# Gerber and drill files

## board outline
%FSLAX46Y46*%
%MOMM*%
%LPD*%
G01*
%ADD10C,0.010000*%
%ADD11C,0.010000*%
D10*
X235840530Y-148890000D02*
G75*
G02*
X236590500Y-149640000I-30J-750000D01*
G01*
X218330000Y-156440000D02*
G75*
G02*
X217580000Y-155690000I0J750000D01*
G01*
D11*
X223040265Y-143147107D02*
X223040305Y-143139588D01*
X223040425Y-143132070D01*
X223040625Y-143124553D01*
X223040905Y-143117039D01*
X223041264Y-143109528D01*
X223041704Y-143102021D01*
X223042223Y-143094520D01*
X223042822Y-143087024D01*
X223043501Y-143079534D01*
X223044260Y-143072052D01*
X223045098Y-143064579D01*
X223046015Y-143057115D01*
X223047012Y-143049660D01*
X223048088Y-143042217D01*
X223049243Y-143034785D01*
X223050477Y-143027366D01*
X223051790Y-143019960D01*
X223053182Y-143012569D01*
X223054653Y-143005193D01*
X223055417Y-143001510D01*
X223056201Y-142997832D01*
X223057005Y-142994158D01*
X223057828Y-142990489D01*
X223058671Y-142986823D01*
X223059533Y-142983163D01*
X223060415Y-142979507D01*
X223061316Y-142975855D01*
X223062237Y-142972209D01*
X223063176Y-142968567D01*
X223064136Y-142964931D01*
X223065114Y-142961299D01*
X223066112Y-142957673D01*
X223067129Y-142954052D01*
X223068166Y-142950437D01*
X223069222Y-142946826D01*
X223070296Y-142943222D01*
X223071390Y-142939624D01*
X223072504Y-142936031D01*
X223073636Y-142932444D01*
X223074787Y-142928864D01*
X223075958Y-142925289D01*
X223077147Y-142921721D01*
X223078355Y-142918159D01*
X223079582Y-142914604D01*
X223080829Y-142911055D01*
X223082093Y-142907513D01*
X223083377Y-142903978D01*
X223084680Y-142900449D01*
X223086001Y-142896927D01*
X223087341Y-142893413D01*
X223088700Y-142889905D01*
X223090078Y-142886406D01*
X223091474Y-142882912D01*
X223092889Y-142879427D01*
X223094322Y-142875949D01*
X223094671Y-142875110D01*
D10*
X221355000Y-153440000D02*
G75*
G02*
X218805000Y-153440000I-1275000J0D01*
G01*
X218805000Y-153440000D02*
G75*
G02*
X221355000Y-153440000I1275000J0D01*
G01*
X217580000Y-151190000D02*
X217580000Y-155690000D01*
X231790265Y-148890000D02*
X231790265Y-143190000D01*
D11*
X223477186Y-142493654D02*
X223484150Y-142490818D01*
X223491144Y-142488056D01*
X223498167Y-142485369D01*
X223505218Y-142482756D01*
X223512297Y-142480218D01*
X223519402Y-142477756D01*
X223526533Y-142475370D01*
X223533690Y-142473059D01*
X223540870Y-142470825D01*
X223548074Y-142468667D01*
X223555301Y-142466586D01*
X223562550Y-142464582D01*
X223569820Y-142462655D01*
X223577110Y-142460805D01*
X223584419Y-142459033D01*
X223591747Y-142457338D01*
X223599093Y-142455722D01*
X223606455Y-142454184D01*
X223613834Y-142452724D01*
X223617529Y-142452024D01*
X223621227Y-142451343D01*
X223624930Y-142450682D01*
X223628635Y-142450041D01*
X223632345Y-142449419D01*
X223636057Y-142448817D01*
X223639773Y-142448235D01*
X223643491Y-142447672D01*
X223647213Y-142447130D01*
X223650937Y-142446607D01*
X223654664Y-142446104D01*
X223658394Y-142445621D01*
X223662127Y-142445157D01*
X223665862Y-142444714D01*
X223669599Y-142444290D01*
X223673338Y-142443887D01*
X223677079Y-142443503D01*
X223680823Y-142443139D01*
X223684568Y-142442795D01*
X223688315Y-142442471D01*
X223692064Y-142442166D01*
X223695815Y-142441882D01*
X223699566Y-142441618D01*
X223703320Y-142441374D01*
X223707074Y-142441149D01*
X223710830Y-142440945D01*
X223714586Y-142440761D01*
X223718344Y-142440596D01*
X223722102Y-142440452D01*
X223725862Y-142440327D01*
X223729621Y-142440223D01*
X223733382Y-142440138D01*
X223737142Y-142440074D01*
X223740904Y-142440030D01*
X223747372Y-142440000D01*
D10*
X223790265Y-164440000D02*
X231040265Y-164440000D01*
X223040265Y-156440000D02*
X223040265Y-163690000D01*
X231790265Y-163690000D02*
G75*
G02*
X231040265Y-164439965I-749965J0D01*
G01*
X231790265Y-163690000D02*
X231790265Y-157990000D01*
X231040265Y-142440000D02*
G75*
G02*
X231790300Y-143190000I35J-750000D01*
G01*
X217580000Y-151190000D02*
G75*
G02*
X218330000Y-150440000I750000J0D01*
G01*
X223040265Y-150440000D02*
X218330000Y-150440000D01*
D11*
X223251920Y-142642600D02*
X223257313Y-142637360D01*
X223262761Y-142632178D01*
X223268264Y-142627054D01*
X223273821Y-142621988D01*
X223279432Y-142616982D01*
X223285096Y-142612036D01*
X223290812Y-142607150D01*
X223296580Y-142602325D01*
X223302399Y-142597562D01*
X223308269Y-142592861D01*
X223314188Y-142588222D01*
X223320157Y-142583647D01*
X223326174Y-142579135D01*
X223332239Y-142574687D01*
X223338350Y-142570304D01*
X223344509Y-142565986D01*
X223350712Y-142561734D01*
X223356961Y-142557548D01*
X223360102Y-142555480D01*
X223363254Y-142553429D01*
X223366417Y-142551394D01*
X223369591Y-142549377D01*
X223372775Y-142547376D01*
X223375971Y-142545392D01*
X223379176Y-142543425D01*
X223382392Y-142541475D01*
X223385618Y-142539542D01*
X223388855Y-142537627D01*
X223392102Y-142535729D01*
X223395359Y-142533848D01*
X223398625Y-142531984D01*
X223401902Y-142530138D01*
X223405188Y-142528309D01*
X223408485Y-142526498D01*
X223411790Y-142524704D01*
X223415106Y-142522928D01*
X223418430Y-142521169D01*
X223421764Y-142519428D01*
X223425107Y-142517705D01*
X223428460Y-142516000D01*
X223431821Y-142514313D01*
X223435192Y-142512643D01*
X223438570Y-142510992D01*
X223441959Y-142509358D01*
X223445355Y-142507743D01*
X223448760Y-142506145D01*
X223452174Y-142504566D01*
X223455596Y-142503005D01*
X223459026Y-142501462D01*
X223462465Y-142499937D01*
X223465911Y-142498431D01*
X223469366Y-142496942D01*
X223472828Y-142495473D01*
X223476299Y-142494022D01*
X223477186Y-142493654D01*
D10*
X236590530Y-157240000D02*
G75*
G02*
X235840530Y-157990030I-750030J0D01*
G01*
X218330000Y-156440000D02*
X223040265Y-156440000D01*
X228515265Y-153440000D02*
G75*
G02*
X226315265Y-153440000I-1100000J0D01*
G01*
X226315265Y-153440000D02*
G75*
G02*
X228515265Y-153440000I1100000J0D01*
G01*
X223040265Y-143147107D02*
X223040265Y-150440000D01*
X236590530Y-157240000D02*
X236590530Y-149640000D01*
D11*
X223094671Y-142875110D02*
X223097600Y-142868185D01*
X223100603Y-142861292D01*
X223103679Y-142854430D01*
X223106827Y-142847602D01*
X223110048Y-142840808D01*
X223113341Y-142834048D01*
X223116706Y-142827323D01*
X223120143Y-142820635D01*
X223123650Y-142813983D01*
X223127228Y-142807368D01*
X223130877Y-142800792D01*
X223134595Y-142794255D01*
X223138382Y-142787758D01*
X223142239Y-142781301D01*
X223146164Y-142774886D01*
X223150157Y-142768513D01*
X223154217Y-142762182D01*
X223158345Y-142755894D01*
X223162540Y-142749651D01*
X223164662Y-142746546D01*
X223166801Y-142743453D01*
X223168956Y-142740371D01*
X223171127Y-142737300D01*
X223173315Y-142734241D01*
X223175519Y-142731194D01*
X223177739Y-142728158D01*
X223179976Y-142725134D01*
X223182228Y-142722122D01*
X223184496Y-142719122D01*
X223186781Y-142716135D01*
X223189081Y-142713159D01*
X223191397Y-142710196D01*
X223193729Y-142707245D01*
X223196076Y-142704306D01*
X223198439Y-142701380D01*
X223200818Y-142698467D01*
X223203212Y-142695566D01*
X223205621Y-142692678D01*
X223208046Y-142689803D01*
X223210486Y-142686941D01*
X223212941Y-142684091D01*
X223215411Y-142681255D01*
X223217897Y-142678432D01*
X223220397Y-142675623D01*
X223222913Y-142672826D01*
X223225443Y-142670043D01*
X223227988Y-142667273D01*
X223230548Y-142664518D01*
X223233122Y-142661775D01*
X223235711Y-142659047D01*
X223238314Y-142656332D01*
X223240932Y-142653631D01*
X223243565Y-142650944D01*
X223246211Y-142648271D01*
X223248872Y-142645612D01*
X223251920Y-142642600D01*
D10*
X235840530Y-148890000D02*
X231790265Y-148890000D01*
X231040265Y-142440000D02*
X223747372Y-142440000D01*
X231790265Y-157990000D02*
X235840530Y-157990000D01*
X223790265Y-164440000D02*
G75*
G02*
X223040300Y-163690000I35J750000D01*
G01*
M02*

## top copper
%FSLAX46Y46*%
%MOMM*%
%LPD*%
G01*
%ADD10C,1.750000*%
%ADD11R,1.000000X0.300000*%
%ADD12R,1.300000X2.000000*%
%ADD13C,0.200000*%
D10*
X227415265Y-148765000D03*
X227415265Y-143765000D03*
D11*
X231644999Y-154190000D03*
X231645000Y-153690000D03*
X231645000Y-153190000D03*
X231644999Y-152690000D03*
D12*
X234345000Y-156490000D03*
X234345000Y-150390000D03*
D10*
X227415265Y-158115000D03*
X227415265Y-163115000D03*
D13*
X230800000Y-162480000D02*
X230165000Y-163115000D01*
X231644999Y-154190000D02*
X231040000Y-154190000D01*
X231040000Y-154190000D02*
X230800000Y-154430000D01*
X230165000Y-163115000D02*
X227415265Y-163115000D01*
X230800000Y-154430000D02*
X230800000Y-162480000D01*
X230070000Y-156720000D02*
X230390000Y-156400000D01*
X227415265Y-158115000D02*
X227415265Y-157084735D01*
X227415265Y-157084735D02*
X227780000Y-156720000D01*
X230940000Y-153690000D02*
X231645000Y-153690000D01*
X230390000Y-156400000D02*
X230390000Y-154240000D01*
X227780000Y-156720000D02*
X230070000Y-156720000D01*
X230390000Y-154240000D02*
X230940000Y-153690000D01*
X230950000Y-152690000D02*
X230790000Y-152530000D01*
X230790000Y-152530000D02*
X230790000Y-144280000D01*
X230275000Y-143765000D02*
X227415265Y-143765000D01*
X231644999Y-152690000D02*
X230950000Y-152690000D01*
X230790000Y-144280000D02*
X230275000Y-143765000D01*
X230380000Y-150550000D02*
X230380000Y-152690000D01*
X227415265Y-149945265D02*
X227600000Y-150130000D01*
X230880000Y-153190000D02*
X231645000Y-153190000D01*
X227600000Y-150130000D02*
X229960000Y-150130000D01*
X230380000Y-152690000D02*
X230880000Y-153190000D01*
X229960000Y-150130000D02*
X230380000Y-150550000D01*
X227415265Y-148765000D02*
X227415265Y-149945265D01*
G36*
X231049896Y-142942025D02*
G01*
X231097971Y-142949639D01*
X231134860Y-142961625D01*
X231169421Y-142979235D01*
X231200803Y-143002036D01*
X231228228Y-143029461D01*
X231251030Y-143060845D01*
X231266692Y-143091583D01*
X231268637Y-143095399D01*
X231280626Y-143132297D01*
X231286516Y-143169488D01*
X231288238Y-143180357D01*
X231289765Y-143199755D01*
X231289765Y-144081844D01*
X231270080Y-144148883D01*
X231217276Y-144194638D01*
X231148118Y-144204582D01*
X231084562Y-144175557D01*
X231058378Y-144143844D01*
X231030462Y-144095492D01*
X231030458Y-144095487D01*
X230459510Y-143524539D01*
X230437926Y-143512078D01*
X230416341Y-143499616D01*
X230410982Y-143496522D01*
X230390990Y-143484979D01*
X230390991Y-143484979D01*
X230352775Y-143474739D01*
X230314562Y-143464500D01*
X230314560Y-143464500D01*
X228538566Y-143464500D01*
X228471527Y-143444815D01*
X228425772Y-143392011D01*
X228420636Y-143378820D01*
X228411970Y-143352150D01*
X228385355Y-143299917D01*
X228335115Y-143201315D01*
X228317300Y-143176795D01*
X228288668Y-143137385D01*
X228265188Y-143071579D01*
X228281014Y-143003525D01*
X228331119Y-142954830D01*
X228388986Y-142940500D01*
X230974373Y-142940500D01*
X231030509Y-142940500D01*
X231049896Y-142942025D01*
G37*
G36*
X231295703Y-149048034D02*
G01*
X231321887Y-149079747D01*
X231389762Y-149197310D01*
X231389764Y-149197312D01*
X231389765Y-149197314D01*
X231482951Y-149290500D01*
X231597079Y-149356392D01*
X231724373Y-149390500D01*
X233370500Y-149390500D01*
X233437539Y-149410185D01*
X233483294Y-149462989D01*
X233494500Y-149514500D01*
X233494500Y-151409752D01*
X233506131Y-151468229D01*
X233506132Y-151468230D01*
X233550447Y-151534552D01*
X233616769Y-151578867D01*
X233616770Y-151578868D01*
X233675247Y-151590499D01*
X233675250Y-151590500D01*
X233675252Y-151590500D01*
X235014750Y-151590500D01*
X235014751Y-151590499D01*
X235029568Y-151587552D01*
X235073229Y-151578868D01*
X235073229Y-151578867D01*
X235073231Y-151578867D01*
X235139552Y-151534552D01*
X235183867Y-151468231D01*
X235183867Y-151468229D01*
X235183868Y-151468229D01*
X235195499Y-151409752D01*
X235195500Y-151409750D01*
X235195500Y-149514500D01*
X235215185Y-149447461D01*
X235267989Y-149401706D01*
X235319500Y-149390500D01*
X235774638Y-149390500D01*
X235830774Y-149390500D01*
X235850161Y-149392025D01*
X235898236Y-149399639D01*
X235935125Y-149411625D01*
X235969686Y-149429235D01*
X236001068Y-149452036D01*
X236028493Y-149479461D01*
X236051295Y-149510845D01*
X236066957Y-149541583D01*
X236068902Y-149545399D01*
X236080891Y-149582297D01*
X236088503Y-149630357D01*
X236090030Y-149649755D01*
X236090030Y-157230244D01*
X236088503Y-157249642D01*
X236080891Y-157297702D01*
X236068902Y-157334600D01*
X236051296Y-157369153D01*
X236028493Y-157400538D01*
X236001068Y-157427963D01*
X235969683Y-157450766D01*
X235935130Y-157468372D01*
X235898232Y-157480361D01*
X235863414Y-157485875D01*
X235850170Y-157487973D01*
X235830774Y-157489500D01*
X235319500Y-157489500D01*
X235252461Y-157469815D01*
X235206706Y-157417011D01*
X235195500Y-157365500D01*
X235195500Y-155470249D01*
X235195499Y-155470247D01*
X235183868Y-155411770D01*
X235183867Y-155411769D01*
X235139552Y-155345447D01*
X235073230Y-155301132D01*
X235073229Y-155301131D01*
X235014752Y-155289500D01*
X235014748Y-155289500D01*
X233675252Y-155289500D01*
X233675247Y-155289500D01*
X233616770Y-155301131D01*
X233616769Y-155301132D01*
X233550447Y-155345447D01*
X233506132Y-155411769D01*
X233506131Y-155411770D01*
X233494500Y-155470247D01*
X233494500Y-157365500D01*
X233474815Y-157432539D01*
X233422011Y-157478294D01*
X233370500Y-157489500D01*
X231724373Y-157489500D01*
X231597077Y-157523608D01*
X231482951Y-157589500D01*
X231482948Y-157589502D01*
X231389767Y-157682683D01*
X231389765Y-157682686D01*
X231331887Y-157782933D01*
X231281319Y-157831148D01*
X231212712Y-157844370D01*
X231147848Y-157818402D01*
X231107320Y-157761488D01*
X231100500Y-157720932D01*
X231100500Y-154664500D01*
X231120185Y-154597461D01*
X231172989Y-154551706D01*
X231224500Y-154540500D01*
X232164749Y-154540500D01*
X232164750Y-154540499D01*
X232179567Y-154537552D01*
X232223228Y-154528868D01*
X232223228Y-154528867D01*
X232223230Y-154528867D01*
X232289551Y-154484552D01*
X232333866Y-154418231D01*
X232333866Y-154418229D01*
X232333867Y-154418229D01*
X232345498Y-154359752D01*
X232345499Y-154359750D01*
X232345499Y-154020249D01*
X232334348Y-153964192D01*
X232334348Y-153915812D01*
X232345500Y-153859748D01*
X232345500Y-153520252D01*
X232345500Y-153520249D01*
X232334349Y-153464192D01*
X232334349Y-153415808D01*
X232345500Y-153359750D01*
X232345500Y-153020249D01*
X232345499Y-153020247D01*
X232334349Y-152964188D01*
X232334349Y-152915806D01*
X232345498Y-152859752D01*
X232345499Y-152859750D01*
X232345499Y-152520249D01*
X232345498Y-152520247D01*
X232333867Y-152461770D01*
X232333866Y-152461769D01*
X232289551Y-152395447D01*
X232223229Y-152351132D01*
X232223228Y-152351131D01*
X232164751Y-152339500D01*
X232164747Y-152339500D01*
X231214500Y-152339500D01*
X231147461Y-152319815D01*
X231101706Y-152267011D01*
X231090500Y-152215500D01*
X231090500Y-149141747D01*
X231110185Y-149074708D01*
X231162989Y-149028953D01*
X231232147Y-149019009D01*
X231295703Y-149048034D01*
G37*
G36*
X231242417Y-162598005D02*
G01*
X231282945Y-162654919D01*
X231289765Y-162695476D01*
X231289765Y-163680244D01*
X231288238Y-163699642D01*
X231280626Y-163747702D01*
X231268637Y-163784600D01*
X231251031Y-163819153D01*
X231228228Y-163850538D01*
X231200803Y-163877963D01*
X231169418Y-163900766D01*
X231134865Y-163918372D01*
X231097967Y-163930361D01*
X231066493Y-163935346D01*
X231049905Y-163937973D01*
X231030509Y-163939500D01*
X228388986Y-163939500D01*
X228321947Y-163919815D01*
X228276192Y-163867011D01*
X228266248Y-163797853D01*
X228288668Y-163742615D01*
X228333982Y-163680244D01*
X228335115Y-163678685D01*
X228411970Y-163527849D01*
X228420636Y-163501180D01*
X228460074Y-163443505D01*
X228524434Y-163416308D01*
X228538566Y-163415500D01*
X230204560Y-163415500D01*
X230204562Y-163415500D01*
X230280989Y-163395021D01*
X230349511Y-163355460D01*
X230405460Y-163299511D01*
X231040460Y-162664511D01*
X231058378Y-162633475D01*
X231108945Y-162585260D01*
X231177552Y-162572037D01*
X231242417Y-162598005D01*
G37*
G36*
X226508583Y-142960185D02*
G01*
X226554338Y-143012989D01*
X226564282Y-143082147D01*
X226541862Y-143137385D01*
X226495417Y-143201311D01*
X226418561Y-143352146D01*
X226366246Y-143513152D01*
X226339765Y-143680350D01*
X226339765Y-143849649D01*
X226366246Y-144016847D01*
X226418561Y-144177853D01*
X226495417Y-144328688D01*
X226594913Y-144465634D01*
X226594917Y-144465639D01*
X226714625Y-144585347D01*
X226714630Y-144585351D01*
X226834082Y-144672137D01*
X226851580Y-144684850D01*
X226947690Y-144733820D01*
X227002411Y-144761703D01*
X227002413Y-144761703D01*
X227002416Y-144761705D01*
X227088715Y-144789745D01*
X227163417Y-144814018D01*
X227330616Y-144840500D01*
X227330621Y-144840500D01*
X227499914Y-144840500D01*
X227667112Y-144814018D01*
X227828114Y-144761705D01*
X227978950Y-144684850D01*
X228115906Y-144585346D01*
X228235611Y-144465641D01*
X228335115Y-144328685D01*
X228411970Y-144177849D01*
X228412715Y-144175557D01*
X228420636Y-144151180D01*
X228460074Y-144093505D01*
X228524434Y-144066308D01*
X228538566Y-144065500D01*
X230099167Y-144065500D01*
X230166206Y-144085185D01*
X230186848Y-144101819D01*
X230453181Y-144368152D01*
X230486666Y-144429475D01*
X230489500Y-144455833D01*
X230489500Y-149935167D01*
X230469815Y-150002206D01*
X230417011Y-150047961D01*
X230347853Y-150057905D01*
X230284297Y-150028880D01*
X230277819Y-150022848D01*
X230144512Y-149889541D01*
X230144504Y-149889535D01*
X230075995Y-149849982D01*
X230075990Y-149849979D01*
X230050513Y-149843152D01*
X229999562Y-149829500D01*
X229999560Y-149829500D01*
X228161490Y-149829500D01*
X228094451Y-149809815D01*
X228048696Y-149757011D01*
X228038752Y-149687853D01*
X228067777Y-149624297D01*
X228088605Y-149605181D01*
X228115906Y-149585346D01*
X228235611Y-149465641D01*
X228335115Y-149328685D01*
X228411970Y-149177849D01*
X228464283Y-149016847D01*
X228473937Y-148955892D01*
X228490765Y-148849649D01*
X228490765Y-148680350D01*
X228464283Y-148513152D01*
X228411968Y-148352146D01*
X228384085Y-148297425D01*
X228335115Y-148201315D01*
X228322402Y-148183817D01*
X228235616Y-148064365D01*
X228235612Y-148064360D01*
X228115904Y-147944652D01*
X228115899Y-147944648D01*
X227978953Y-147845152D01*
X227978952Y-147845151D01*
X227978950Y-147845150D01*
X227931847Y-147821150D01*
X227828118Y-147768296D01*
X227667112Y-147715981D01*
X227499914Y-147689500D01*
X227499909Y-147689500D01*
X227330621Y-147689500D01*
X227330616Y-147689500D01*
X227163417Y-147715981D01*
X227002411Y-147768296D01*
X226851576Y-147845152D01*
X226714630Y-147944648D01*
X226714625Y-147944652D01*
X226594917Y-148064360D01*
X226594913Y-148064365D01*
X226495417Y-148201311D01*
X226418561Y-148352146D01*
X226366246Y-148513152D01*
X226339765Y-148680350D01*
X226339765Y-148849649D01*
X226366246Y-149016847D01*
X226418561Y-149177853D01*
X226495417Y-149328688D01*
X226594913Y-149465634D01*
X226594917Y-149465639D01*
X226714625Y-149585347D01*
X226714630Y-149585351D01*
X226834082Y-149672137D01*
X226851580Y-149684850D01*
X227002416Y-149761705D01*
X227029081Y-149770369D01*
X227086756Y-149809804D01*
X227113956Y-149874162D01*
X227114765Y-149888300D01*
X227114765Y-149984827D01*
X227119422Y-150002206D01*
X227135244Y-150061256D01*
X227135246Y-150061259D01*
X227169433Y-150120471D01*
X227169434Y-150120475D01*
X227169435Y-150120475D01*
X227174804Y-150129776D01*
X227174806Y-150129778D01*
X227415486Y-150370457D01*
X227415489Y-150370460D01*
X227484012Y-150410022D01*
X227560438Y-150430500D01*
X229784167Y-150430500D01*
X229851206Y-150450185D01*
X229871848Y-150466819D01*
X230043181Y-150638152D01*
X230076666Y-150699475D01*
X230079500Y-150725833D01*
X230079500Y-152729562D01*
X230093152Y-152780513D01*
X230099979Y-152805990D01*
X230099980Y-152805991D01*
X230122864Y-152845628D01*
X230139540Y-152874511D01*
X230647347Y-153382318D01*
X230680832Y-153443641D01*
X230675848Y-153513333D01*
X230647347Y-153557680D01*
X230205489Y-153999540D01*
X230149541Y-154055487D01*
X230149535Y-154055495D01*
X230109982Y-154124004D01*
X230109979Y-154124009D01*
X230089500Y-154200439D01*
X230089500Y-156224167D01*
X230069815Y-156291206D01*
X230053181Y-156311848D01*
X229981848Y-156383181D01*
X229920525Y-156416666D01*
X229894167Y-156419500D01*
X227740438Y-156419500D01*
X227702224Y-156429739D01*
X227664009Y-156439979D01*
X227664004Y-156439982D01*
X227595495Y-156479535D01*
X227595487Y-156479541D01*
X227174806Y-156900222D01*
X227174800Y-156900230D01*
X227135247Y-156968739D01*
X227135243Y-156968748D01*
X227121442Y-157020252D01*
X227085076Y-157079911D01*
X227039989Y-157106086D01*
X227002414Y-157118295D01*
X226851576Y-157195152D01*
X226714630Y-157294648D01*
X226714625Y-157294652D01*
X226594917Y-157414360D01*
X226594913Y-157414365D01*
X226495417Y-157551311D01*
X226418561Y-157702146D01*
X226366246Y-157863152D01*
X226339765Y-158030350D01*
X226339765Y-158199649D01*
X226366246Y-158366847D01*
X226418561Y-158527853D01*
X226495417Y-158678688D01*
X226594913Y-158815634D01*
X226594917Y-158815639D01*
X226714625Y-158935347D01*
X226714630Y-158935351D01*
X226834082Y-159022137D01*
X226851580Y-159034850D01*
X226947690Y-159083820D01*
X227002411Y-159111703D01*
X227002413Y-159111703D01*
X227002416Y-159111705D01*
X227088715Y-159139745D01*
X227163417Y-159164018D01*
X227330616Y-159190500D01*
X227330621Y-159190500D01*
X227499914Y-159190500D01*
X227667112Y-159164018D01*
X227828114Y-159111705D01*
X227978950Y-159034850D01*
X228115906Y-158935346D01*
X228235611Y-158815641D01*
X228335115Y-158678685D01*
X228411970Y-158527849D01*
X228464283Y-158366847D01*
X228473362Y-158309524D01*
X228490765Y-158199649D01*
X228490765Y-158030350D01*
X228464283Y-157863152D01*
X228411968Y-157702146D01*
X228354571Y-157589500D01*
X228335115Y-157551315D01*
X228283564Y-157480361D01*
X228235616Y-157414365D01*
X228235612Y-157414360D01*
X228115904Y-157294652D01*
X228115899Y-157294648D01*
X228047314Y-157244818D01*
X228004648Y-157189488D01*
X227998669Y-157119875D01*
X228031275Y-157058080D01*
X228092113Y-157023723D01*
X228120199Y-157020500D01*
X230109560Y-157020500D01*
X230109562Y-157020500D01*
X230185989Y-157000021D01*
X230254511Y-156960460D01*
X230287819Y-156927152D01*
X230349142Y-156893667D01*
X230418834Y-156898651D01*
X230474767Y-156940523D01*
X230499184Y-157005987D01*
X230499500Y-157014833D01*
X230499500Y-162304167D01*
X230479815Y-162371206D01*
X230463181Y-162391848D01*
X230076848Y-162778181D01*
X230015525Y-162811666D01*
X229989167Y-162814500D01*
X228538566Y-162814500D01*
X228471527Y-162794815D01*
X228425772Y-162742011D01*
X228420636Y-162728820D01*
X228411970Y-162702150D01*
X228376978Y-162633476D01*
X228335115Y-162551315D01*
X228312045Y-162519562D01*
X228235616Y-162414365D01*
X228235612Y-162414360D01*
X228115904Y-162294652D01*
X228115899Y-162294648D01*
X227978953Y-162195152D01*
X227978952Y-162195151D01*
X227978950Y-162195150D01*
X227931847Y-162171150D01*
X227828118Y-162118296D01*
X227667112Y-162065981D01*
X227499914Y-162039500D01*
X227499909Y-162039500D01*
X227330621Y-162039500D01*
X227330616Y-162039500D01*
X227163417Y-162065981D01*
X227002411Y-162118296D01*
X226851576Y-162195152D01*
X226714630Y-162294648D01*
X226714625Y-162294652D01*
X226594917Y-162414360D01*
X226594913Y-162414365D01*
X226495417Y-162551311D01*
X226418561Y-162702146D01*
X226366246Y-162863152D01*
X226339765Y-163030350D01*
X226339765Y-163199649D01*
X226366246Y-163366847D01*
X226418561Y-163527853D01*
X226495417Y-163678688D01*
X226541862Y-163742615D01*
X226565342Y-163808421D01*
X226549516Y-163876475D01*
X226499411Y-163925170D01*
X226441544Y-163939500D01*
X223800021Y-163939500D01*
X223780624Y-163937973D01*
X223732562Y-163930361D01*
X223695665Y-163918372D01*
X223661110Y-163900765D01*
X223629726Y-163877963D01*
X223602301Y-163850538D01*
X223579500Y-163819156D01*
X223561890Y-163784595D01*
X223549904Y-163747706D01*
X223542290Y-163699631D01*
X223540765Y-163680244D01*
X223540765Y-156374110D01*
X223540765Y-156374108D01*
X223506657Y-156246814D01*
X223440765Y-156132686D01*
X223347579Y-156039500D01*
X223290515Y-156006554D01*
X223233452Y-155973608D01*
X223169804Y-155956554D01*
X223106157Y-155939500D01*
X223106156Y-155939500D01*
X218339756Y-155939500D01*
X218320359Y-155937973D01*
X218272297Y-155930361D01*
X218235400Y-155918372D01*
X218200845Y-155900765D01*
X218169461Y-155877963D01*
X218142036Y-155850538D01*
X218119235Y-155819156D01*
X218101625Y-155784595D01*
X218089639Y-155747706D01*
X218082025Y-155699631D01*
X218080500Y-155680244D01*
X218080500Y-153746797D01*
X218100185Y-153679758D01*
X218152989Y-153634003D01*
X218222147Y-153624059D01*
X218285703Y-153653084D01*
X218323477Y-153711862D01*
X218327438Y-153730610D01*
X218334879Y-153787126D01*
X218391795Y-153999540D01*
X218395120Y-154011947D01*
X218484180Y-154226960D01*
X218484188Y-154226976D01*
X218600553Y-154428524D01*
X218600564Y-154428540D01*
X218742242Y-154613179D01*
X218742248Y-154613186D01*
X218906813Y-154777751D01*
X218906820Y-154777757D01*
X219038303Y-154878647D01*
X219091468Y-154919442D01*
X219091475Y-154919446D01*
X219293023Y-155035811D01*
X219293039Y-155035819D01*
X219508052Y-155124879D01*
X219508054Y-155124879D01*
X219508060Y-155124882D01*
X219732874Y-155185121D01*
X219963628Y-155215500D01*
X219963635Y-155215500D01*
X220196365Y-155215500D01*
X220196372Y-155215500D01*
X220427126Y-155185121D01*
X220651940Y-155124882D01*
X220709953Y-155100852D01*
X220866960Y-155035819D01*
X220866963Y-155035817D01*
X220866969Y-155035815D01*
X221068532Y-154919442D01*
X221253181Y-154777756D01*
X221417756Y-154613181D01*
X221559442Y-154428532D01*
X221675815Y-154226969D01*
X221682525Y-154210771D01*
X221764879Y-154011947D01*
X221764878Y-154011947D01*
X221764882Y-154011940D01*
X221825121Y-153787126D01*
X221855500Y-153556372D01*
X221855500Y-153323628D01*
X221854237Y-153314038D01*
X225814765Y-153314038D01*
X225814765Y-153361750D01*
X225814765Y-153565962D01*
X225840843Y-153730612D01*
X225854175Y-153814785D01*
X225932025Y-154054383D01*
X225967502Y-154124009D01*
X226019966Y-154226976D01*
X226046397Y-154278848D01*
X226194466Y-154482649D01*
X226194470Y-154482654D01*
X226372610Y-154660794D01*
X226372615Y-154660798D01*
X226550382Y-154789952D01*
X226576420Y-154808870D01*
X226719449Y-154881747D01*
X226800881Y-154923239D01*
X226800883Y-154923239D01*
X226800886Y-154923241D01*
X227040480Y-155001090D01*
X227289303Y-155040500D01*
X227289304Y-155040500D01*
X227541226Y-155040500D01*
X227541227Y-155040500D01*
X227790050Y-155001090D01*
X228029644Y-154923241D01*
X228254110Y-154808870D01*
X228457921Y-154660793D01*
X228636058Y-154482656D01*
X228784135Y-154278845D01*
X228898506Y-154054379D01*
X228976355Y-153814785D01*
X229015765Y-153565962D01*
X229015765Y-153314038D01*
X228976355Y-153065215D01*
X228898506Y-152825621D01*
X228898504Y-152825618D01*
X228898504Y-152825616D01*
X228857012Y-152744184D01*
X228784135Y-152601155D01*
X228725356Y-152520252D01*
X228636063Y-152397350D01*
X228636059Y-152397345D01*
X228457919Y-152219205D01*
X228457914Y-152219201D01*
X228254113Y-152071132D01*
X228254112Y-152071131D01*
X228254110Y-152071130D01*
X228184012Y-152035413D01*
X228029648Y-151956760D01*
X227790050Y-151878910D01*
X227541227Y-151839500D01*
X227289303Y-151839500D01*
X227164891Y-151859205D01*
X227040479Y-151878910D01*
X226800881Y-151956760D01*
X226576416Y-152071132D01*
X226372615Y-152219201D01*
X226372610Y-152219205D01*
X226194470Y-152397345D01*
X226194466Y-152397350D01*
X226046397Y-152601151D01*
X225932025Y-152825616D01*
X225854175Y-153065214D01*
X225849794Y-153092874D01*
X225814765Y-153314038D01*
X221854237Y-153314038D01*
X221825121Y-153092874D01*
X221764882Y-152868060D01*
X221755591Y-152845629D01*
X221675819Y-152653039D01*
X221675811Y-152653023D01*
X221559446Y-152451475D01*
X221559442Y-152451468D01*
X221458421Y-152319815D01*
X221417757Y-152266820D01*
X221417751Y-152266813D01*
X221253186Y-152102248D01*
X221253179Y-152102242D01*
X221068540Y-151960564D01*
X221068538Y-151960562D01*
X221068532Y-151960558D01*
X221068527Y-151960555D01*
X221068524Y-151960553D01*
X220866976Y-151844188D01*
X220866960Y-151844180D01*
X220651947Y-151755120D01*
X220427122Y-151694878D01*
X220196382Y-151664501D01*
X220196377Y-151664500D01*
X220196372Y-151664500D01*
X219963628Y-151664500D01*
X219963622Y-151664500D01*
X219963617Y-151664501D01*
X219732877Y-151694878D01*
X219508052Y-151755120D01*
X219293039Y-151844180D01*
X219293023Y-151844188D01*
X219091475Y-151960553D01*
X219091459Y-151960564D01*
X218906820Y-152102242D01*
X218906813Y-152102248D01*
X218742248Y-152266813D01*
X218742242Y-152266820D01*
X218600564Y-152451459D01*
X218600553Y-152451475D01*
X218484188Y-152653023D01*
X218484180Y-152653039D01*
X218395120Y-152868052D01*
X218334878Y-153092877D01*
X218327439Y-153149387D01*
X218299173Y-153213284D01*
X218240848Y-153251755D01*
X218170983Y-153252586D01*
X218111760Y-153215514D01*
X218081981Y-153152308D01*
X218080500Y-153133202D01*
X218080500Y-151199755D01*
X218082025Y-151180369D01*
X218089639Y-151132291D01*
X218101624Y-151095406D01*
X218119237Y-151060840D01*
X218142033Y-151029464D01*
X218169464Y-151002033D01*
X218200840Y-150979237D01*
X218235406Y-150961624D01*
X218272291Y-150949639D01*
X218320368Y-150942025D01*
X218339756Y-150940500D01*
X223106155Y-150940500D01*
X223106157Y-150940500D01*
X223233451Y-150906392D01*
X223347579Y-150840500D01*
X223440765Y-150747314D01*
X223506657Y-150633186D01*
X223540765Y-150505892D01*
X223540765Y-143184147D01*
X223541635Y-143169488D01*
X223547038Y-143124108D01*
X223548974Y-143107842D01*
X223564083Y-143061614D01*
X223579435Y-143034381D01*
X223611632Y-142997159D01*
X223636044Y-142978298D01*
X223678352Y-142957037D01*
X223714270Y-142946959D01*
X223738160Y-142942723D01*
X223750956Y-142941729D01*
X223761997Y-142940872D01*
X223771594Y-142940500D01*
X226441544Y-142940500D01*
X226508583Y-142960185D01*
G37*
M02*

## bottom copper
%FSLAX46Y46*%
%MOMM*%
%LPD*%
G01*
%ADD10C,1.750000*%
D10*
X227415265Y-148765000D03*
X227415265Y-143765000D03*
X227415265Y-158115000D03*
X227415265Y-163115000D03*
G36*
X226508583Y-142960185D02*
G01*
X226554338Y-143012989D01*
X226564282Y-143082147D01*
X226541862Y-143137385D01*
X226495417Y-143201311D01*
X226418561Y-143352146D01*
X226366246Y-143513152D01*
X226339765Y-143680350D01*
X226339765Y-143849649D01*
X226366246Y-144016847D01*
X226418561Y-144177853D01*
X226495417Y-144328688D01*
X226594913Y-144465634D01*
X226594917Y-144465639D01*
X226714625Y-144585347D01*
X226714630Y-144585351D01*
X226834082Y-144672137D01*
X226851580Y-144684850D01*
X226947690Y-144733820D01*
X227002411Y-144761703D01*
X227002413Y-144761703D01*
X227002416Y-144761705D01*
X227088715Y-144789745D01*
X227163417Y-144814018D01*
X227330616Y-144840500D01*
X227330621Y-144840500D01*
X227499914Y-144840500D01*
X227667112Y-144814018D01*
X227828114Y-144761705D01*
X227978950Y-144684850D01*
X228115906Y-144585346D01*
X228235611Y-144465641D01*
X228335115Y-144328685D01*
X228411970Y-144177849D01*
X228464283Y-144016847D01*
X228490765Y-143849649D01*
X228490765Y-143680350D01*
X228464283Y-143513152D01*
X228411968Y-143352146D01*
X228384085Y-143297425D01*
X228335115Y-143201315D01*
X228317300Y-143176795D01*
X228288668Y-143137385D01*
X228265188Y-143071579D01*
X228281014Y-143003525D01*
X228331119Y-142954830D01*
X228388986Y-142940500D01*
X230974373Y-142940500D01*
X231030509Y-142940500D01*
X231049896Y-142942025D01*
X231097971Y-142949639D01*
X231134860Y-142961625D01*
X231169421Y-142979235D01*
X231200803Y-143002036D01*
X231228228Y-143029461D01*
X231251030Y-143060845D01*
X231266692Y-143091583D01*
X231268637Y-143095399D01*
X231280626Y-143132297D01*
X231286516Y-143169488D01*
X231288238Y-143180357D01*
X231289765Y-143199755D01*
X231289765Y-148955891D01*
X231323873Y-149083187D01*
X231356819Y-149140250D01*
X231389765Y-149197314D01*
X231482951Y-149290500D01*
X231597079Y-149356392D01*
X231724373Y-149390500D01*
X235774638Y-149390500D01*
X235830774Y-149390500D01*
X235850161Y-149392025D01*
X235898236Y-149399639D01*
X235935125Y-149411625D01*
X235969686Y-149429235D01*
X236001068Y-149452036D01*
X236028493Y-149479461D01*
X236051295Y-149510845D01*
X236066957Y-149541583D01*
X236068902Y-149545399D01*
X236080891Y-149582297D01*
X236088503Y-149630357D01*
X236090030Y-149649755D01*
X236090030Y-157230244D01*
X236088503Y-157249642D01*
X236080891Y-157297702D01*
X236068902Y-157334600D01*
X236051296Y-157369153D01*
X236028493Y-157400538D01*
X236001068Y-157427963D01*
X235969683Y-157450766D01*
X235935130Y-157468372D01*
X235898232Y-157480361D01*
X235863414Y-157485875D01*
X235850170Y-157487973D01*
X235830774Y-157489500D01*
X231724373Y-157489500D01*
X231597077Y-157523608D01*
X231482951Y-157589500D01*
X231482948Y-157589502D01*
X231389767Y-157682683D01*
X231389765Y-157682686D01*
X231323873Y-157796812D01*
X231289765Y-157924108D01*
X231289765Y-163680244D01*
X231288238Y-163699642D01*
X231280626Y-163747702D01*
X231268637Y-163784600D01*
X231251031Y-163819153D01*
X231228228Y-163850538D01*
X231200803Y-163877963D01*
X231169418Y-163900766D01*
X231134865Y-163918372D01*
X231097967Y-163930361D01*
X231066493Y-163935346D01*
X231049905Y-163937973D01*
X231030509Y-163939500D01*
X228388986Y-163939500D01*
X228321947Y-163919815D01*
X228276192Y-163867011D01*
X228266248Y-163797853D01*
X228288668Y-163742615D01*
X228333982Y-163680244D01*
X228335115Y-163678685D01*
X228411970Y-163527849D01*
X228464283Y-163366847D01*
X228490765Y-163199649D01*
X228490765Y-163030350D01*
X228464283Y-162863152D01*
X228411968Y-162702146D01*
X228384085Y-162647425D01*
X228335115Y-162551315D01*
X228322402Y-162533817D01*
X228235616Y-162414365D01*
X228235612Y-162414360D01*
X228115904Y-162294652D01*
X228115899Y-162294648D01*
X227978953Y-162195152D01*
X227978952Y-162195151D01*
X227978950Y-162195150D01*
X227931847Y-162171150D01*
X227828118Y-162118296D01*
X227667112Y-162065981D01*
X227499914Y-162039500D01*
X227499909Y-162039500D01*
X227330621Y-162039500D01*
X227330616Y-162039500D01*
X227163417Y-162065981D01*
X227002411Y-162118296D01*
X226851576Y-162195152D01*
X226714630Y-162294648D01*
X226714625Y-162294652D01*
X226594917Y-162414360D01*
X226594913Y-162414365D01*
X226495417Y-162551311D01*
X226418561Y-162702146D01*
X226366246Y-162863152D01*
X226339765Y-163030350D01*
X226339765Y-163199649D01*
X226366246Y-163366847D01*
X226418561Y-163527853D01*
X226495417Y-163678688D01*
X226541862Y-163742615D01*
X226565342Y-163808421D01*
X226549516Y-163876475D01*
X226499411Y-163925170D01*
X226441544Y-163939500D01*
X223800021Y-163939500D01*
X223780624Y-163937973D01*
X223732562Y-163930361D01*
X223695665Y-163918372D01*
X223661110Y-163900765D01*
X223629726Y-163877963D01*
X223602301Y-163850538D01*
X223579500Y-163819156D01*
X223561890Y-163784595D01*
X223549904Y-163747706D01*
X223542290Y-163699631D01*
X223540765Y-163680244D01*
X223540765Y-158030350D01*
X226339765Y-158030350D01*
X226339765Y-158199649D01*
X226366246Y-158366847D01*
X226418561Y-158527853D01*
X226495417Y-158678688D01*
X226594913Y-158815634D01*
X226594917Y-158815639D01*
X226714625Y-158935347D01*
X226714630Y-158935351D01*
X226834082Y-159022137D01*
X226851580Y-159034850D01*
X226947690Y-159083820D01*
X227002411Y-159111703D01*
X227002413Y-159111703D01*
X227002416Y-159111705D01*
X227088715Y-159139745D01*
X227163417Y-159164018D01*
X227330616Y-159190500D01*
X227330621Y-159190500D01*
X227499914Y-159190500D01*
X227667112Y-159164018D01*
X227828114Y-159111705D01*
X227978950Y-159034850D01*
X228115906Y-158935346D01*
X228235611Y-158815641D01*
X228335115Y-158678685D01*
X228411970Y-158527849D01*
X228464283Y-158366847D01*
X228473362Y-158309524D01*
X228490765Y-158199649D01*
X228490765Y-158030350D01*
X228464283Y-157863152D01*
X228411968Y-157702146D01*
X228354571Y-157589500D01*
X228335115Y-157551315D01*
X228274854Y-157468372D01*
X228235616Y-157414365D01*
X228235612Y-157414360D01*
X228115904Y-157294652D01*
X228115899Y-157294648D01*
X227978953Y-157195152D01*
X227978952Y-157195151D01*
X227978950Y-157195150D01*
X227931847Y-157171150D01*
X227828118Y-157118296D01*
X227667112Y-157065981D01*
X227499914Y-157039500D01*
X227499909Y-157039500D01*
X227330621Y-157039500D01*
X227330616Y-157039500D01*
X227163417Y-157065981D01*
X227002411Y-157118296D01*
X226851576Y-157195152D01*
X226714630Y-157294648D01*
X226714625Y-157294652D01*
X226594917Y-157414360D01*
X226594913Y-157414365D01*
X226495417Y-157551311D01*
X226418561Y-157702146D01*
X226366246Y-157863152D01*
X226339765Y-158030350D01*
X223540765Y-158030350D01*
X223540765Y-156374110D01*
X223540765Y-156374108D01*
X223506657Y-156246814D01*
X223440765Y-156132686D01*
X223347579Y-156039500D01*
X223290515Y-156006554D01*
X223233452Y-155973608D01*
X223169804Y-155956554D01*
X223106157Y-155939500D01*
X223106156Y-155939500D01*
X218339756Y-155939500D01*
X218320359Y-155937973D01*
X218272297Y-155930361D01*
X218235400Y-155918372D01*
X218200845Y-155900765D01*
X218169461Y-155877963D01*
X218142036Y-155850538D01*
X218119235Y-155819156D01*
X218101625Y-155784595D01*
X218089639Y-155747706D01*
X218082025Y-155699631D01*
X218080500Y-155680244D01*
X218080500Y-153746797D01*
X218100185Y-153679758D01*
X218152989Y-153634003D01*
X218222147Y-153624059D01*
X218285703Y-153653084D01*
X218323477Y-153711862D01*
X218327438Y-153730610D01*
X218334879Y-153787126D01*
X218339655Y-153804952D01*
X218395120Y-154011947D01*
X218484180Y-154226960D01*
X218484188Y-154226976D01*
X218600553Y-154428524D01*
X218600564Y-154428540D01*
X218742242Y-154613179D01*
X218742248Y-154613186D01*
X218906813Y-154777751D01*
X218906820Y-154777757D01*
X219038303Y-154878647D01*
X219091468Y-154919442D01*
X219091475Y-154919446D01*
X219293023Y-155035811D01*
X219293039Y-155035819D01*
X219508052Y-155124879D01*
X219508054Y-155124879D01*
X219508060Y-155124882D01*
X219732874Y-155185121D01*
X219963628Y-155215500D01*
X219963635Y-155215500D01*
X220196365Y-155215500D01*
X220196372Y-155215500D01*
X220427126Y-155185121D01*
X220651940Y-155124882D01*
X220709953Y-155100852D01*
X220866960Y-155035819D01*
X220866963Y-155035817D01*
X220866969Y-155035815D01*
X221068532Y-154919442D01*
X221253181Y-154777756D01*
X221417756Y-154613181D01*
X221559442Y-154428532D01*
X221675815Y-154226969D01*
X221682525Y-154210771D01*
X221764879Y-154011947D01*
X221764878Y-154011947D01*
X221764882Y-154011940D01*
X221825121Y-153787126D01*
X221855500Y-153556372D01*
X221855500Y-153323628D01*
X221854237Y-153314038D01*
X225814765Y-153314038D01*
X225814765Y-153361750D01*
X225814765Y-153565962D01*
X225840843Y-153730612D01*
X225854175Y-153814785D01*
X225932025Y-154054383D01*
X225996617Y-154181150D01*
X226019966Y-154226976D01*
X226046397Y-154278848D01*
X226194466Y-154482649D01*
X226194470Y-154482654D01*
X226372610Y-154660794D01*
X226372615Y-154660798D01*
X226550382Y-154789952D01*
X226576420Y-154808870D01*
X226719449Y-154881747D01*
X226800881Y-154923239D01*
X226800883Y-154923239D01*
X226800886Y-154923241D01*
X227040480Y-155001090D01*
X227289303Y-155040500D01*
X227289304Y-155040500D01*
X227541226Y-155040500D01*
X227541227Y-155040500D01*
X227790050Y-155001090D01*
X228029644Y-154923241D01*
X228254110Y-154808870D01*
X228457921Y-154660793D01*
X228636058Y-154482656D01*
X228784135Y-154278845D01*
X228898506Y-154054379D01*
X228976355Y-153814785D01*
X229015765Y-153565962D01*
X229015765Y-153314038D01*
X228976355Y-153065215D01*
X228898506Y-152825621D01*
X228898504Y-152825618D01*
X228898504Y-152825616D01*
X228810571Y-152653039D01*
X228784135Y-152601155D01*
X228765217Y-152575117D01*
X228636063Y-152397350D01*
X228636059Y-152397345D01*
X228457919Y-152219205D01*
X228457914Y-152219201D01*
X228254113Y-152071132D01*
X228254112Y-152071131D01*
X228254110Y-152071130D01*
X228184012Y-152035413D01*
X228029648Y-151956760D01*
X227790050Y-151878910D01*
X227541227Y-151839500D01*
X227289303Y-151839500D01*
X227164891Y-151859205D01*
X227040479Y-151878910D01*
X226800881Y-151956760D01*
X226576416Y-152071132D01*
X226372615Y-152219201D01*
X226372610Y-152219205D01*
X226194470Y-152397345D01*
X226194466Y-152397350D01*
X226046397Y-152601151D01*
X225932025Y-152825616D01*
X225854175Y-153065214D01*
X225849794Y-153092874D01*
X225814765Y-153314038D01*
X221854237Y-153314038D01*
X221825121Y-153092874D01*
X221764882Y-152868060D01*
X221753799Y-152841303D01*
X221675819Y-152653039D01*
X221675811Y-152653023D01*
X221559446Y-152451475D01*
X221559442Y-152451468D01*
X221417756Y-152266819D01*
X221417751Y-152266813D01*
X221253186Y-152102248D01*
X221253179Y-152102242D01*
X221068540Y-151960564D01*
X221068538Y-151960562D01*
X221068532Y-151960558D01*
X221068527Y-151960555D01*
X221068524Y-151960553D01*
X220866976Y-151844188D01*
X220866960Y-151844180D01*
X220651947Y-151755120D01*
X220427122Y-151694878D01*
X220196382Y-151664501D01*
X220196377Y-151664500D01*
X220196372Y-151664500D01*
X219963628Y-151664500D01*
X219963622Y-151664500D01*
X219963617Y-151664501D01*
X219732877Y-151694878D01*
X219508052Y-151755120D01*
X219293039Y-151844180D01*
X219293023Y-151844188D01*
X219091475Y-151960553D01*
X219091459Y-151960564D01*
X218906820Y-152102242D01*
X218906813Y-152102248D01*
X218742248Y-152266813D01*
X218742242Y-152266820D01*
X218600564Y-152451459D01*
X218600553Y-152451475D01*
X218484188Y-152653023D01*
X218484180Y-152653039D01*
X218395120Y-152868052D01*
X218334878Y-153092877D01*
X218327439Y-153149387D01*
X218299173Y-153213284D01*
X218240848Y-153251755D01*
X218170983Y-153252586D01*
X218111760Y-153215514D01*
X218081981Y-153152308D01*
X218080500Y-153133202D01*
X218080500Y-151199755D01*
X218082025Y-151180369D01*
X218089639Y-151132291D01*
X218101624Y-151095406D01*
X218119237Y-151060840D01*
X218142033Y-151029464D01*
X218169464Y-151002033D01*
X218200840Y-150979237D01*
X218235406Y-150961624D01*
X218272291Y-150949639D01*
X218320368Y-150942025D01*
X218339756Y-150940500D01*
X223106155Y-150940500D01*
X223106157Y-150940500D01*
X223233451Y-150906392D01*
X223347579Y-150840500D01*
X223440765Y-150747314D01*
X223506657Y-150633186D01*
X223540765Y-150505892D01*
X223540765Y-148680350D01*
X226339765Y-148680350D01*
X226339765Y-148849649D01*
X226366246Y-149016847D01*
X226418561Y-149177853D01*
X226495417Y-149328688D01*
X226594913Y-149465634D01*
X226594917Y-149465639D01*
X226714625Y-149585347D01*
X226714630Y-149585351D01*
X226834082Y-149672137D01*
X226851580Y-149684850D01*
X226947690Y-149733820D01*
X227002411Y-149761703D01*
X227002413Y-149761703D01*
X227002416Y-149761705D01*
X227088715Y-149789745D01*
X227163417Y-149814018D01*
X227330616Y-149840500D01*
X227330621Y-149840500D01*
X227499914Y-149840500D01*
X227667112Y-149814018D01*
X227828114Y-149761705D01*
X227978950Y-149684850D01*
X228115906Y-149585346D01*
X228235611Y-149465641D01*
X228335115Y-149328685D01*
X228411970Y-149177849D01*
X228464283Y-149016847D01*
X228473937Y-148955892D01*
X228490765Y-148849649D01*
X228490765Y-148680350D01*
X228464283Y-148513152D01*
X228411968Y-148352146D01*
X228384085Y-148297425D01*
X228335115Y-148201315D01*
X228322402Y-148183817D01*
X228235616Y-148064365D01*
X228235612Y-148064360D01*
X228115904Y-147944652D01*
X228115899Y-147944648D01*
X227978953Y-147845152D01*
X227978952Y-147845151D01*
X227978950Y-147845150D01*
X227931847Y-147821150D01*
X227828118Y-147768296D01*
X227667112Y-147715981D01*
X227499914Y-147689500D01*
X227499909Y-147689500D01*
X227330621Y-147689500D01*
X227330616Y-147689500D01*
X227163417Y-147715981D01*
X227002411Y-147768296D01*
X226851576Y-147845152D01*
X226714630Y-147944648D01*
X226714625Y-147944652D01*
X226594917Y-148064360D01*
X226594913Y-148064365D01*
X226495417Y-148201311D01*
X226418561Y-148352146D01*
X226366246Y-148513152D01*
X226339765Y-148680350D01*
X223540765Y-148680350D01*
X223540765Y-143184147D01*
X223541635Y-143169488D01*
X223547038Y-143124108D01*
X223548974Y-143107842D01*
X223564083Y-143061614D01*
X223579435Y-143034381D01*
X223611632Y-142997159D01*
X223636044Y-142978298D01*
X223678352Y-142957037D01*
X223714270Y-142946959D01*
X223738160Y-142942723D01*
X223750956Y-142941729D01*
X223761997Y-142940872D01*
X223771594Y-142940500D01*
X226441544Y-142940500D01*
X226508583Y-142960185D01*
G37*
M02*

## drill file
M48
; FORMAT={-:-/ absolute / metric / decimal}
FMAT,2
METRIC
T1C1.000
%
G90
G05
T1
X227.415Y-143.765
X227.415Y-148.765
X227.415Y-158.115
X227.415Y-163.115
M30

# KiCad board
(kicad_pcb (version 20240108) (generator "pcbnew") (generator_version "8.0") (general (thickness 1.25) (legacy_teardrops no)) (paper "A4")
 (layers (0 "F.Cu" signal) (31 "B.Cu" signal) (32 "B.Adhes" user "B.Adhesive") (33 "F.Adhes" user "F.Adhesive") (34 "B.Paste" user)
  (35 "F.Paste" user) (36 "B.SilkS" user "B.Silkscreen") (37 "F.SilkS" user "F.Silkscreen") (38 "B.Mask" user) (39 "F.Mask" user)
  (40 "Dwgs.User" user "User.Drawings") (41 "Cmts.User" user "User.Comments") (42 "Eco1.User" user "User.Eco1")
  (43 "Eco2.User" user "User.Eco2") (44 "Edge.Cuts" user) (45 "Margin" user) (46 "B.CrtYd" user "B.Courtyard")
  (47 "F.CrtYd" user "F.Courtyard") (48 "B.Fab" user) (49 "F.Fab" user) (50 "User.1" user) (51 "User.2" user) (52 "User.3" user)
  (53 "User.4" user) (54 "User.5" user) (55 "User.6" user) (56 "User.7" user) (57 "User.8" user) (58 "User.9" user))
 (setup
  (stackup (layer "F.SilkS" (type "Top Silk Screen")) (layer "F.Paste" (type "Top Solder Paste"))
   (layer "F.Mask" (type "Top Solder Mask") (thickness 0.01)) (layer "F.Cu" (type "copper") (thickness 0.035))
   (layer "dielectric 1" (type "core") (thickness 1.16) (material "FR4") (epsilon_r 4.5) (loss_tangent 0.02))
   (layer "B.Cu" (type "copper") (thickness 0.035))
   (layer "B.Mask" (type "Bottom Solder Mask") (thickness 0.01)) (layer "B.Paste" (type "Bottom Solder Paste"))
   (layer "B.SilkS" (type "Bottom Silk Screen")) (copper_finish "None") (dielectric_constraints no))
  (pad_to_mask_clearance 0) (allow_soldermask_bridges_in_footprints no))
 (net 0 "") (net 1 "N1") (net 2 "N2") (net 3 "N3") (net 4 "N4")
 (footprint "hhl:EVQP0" (layer "F.Cu") (at 227.415265 146.265)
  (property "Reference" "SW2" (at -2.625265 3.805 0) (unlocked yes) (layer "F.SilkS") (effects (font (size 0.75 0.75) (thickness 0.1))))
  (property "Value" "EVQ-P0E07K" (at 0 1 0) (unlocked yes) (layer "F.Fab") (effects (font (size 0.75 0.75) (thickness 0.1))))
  (pad "1" thru_hole circle (at 0 2.5) (size 1.75 1.75) (drill 1) (layers "*.Cu" "*.Mask" "B.Paste") (remove_unused_layers no) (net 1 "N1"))
  (pad "2" thru_hole circle (at 0 -2.5) (size 1.75 1.75) (drill 1) (layers "*.Cu" "*.Mask" "B.Paste") (remove_unused_layers no) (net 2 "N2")))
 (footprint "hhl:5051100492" (layer "F.Cu") (at 233.87 153.44 90)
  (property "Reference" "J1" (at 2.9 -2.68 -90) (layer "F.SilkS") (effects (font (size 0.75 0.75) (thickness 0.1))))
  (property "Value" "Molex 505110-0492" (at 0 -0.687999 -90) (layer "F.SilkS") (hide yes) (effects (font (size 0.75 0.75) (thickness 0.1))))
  (pad "1" smd rect (at -0.75 -2.225001 90) (size 0.3 1) (layers "F.Cu" "F.Paste" "F.Mask") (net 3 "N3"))
  (pad "2" smd rect (at -0.25 -2.225 90) (size 0.3 1) (layers "F.Cu" "F.Paste" "F.Mask") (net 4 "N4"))
  (pad "3" smd rect (at 0.25 -2.225 90) (size 0.3 1) (layers "F.Cu" "F.Paste" "F.Mask") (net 1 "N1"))
  (pad "4" smd rect (at 0.75 -2.225001 90) (size 0.3 1) (layers "F.Cu" "F.Paste" "F.Mask") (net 2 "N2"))
  (pad "MP1" smd rect (at -3.05 0.475 180) (size 1.3 2) (layers "F.Cu" "F.Paste" "F.Mask"))
  (pad "MP2" smd rect (at 3.05 0.475 180) (size 1.3 2) (layers "F.Cu" "F.Paste" "F.Mask")))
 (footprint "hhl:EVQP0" (layer "F.Cu") (at 227.415265 160.615 180)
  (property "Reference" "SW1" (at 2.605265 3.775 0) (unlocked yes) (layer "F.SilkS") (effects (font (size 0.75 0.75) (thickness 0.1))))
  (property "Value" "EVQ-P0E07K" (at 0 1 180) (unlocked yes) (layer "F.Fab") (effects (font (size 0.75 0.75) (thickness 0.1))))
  (pad "1" thru_hole circle (at 0 2.5 180) (size 1.75 1.75) (drill 1) (layers "*.Cu" "*.Mask" "B.Paste") (remove_unused_layers no)
   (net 4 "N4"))
  (pad "2" thru_hole circle (at 0 -2.5 180) (size 1.75 1.75) (drill 1) (layers "*.Cu" "*.Mask" "B.Paste") (remove_unused_layers no)
   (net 3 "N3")))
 (gr_arc (start 235.84053 148.89) (mid 236.37086 149.10967) (end 236.59053 149.64) (stroke (width 0.01) (type default)) (layer "Edge.Cuts"))
 (gr_arc (start 218.33 156.44) (mid 217.79967 156.22033) (end 217.58 155.69) (stroke (width 0.01) (type default)) (layer "Edge.Cuts"))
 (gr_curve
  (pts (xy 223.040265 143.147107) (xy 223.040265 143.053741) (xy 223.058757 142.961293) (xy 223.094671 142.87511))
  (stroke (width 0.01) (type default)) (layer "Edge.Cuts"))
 (gr_circle (center 220.08 153.44) (end 221.355 153.44) (stroke (width 0.01) (type default)) (fill none) (layer "Edge.Cuts"))
 (gr_line (start 217.58 151.19) (end 217.58 155.69) (stroke (width 0.01) (type default)) (layer "Edge.Cuts"))
 (gr_line (start 231.790265 148.89) (end 231.790265 143.19) (stroke (width 0.01) (type default)) (layer "Edge.Cuts"))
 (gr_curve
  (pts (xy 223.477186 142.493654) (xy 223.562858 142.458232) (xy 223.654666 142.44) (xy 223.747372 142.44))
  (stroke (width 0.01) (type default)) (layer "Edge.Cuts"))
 (gr_line (start 223.790265 164.44) (end 231.040265 164.44) (stroke (width 0.01) (type default)) (layer "Edge.Cuts"))
 (gr_line (start 223.040265 156.44) (end 223.040265 163.69) (stroke (width 0.01) (type default)) (layer "Edge.Cuts"))
 (gr_arc (start 231.790265 163.69) (mid 231.570595 164.22033) (end 231.040265 164.44) (stroke (width 0.01) (type default))
  (layer "Edge.Cuts"))
 (gr_line (start 231.790265 163.69) (end 231.790265 157.99) (stroke (width 0.01) (type default)) (layer "Edge.Cuts"))
 (gr_arc (start 231.040265 142.44) (mid 231.570595 142.65967) (end 231.790265 143.19) (stroke (width 0.01) (type default))
  (layer "Edge.Cuts"))
 (gr_arc (start 217.58 151.19) (mid 217.79967 150.65967) (end 218.33 150.44) (stroke (width 0.01) (type default)) (layer "Edge.Cuts"))
 (gr_line (start 223.040265 150.44) (end 218.33 150.44) (stroke (width 0.01) (type default)) (layer "Edge.Cuts"))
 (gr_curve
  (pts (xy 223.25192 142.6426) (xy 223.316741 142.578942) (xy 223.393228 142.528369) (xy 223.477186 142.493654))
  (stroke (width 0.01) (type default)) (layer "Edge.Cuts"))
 (gr_arc (start 236.59053 157.24) (mid 236.37086 157.77033) (end 235.84053 157.99) (stroke (width 0.01) (type default)) (layer "Edge.Cuts"))
 (gr_line (start 218.33 156.44) (end 223.040265 156.44) (stroke (width 0.01) (type default)) (layer "Edge.Cuts"))
 (gr_circle (center 227.415265 153.44) (end 228.515265 153.44) (stroke (width 0.01) (type default)) (fill none) (layer "Edge.Cuts"))
 (gr_line (start 223.040265 143.147107) (end 223.040265 150.44) (stroke (width 0.01) (type default)) (layer "Edge.Cuts"))
 (gr_line (start 236.59053 157.24) (end 236.59053 149.64) (stroke (width 0.01) (type default)) (layer "Edge.Cuts"))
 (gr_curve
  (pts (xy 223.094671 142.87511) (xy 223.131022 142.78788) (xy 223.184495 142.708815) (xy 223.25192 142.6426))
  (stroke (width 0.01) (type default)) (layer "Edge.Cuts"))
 (gr_line (start 235.84053 148.89) (end 231.790265 148.89) (stroke (width 0.01) (type default)) (layer "Edge.Cuts"))
 (gr_line (start 231.040265 142.44) (end 223.747372 142.44) (stroke (width 0.01) (type default)) (layer "Edge.Cuts"))
 (gr_line (start 231.790265 157.99) (end 235.84053 157.99) (stroke (width 0.01) (type default)) (layer "Edge.Cuts"))
 (gr_arc (start 223.790265 164.44) (mid 223.259935 164.22033) (end 223.040265 163.69) (stroke (width 0.01) (type default))
  (layer "Edge.Cuts"))
 (segment (start 230.8 162.48) (end 230.165 163.115) (width 0.2) (layer "F.Cu") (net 3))
 (segment (start 231.644999 154.19) (end 231.04 154.19) (width 0.2) (layer "F.Cu") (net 3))
 (segment (start 231.04 154.19) (end 230.8 154.43) (width 0.2) (layer "F.Cu") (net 3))
 (segment (start 230.165 163.115) (end 227.415265 163.115) (width 0.2) (layer "F.Cu") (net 3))
 (segment (start 230.8 154.43) (end 230.8 162.48) (width 0.2) (layer "F.Cu") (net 3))
 (segment (start 230.07 156.72) (end 230.39 156.4) (width 0.2) (layer "F.Cu") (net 4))
 (segment (start 227.415265 158.115) (end 227.415265 157.084735) (width 0.2) (layer "F.Cu") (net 4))
 (segment (start 227.415265 157.084735) (end 227.78 156.72) (width 0.2) (layer "F.Cu") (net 4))
 (segment (start 230.94 153.69) (end 231.645 153.69) (width 0.2) (layer "F.Cu") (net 4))
 (segment (start 230.39 156.4) (end 230.39 154.24) (width 0.2) (layer "F.Cu") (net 4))
 (segment (start 227.78 156.72) (end 230.07 156.72) (width 0.2) (layer "F.Cu") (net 4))
 (segment (start 230.39 154.24) (end 230.94 153.69) (width 0.2) (layer "F.Cu") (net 4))
 (segment (start 230.95 152.69) (end 230.79 152.53) (width 0.2) (layer "F.Cu") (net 2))
 (segment (start 230.79 152.53) (end 230.79 144.28) (width 0.2) (layer "F.Cu") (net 2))
 (segment (start 230.275 143.765) (end 227.415265 143.765) (width 0.2) (layer "F.Cu") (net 2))
 (segment (start 231.644999 152.69) (end 230.95 152.69) (width 0.2) (layer "F.Cu") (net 2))
 (segment (start 230.79 144.28) (end 230.275 143.765) (width 0.2) (layer "F.Cu") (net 2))
 (segment (start 230.38 150.55) (end 230.38 152.69) (width 0.2) (layer "F.Cu") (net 1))
 (segment (start 227.415265 149.945265) (end 227.6 150.13) (width 0.2) (layer "F.Cu") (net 1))
 (segment (start 230.88 153.19) (end 231.645 153.19) (width 0.2) (layer "F.Cu") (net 1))
 (segment (start 227.6 150.13) (end 229.96 150.13) (width 0.2) (layer "F.Cu") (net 1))
 (segment (start 230.38 152.69) (end 230.88 153.19) (width 0.2) (layer "F.Cu") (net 1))
 (segment (start 229.96 150.13) (end 230.38 150.55) (width 0.2) (layer "F.Cu") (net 1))
 (segment (start 227.415265 148.765) (end 227.415265 149.945265) (width 0.2) (layer "F.Cu") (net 1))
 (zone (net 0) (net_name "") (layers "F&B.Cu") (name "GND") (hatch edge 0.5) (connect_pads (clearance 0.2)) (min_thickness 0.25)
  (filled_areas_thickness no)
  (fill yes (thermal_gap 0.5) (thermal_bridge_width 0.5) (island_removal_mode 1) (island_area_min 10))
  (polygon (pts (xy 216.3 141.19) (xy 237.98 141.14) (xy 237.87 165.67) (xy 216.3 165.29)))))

